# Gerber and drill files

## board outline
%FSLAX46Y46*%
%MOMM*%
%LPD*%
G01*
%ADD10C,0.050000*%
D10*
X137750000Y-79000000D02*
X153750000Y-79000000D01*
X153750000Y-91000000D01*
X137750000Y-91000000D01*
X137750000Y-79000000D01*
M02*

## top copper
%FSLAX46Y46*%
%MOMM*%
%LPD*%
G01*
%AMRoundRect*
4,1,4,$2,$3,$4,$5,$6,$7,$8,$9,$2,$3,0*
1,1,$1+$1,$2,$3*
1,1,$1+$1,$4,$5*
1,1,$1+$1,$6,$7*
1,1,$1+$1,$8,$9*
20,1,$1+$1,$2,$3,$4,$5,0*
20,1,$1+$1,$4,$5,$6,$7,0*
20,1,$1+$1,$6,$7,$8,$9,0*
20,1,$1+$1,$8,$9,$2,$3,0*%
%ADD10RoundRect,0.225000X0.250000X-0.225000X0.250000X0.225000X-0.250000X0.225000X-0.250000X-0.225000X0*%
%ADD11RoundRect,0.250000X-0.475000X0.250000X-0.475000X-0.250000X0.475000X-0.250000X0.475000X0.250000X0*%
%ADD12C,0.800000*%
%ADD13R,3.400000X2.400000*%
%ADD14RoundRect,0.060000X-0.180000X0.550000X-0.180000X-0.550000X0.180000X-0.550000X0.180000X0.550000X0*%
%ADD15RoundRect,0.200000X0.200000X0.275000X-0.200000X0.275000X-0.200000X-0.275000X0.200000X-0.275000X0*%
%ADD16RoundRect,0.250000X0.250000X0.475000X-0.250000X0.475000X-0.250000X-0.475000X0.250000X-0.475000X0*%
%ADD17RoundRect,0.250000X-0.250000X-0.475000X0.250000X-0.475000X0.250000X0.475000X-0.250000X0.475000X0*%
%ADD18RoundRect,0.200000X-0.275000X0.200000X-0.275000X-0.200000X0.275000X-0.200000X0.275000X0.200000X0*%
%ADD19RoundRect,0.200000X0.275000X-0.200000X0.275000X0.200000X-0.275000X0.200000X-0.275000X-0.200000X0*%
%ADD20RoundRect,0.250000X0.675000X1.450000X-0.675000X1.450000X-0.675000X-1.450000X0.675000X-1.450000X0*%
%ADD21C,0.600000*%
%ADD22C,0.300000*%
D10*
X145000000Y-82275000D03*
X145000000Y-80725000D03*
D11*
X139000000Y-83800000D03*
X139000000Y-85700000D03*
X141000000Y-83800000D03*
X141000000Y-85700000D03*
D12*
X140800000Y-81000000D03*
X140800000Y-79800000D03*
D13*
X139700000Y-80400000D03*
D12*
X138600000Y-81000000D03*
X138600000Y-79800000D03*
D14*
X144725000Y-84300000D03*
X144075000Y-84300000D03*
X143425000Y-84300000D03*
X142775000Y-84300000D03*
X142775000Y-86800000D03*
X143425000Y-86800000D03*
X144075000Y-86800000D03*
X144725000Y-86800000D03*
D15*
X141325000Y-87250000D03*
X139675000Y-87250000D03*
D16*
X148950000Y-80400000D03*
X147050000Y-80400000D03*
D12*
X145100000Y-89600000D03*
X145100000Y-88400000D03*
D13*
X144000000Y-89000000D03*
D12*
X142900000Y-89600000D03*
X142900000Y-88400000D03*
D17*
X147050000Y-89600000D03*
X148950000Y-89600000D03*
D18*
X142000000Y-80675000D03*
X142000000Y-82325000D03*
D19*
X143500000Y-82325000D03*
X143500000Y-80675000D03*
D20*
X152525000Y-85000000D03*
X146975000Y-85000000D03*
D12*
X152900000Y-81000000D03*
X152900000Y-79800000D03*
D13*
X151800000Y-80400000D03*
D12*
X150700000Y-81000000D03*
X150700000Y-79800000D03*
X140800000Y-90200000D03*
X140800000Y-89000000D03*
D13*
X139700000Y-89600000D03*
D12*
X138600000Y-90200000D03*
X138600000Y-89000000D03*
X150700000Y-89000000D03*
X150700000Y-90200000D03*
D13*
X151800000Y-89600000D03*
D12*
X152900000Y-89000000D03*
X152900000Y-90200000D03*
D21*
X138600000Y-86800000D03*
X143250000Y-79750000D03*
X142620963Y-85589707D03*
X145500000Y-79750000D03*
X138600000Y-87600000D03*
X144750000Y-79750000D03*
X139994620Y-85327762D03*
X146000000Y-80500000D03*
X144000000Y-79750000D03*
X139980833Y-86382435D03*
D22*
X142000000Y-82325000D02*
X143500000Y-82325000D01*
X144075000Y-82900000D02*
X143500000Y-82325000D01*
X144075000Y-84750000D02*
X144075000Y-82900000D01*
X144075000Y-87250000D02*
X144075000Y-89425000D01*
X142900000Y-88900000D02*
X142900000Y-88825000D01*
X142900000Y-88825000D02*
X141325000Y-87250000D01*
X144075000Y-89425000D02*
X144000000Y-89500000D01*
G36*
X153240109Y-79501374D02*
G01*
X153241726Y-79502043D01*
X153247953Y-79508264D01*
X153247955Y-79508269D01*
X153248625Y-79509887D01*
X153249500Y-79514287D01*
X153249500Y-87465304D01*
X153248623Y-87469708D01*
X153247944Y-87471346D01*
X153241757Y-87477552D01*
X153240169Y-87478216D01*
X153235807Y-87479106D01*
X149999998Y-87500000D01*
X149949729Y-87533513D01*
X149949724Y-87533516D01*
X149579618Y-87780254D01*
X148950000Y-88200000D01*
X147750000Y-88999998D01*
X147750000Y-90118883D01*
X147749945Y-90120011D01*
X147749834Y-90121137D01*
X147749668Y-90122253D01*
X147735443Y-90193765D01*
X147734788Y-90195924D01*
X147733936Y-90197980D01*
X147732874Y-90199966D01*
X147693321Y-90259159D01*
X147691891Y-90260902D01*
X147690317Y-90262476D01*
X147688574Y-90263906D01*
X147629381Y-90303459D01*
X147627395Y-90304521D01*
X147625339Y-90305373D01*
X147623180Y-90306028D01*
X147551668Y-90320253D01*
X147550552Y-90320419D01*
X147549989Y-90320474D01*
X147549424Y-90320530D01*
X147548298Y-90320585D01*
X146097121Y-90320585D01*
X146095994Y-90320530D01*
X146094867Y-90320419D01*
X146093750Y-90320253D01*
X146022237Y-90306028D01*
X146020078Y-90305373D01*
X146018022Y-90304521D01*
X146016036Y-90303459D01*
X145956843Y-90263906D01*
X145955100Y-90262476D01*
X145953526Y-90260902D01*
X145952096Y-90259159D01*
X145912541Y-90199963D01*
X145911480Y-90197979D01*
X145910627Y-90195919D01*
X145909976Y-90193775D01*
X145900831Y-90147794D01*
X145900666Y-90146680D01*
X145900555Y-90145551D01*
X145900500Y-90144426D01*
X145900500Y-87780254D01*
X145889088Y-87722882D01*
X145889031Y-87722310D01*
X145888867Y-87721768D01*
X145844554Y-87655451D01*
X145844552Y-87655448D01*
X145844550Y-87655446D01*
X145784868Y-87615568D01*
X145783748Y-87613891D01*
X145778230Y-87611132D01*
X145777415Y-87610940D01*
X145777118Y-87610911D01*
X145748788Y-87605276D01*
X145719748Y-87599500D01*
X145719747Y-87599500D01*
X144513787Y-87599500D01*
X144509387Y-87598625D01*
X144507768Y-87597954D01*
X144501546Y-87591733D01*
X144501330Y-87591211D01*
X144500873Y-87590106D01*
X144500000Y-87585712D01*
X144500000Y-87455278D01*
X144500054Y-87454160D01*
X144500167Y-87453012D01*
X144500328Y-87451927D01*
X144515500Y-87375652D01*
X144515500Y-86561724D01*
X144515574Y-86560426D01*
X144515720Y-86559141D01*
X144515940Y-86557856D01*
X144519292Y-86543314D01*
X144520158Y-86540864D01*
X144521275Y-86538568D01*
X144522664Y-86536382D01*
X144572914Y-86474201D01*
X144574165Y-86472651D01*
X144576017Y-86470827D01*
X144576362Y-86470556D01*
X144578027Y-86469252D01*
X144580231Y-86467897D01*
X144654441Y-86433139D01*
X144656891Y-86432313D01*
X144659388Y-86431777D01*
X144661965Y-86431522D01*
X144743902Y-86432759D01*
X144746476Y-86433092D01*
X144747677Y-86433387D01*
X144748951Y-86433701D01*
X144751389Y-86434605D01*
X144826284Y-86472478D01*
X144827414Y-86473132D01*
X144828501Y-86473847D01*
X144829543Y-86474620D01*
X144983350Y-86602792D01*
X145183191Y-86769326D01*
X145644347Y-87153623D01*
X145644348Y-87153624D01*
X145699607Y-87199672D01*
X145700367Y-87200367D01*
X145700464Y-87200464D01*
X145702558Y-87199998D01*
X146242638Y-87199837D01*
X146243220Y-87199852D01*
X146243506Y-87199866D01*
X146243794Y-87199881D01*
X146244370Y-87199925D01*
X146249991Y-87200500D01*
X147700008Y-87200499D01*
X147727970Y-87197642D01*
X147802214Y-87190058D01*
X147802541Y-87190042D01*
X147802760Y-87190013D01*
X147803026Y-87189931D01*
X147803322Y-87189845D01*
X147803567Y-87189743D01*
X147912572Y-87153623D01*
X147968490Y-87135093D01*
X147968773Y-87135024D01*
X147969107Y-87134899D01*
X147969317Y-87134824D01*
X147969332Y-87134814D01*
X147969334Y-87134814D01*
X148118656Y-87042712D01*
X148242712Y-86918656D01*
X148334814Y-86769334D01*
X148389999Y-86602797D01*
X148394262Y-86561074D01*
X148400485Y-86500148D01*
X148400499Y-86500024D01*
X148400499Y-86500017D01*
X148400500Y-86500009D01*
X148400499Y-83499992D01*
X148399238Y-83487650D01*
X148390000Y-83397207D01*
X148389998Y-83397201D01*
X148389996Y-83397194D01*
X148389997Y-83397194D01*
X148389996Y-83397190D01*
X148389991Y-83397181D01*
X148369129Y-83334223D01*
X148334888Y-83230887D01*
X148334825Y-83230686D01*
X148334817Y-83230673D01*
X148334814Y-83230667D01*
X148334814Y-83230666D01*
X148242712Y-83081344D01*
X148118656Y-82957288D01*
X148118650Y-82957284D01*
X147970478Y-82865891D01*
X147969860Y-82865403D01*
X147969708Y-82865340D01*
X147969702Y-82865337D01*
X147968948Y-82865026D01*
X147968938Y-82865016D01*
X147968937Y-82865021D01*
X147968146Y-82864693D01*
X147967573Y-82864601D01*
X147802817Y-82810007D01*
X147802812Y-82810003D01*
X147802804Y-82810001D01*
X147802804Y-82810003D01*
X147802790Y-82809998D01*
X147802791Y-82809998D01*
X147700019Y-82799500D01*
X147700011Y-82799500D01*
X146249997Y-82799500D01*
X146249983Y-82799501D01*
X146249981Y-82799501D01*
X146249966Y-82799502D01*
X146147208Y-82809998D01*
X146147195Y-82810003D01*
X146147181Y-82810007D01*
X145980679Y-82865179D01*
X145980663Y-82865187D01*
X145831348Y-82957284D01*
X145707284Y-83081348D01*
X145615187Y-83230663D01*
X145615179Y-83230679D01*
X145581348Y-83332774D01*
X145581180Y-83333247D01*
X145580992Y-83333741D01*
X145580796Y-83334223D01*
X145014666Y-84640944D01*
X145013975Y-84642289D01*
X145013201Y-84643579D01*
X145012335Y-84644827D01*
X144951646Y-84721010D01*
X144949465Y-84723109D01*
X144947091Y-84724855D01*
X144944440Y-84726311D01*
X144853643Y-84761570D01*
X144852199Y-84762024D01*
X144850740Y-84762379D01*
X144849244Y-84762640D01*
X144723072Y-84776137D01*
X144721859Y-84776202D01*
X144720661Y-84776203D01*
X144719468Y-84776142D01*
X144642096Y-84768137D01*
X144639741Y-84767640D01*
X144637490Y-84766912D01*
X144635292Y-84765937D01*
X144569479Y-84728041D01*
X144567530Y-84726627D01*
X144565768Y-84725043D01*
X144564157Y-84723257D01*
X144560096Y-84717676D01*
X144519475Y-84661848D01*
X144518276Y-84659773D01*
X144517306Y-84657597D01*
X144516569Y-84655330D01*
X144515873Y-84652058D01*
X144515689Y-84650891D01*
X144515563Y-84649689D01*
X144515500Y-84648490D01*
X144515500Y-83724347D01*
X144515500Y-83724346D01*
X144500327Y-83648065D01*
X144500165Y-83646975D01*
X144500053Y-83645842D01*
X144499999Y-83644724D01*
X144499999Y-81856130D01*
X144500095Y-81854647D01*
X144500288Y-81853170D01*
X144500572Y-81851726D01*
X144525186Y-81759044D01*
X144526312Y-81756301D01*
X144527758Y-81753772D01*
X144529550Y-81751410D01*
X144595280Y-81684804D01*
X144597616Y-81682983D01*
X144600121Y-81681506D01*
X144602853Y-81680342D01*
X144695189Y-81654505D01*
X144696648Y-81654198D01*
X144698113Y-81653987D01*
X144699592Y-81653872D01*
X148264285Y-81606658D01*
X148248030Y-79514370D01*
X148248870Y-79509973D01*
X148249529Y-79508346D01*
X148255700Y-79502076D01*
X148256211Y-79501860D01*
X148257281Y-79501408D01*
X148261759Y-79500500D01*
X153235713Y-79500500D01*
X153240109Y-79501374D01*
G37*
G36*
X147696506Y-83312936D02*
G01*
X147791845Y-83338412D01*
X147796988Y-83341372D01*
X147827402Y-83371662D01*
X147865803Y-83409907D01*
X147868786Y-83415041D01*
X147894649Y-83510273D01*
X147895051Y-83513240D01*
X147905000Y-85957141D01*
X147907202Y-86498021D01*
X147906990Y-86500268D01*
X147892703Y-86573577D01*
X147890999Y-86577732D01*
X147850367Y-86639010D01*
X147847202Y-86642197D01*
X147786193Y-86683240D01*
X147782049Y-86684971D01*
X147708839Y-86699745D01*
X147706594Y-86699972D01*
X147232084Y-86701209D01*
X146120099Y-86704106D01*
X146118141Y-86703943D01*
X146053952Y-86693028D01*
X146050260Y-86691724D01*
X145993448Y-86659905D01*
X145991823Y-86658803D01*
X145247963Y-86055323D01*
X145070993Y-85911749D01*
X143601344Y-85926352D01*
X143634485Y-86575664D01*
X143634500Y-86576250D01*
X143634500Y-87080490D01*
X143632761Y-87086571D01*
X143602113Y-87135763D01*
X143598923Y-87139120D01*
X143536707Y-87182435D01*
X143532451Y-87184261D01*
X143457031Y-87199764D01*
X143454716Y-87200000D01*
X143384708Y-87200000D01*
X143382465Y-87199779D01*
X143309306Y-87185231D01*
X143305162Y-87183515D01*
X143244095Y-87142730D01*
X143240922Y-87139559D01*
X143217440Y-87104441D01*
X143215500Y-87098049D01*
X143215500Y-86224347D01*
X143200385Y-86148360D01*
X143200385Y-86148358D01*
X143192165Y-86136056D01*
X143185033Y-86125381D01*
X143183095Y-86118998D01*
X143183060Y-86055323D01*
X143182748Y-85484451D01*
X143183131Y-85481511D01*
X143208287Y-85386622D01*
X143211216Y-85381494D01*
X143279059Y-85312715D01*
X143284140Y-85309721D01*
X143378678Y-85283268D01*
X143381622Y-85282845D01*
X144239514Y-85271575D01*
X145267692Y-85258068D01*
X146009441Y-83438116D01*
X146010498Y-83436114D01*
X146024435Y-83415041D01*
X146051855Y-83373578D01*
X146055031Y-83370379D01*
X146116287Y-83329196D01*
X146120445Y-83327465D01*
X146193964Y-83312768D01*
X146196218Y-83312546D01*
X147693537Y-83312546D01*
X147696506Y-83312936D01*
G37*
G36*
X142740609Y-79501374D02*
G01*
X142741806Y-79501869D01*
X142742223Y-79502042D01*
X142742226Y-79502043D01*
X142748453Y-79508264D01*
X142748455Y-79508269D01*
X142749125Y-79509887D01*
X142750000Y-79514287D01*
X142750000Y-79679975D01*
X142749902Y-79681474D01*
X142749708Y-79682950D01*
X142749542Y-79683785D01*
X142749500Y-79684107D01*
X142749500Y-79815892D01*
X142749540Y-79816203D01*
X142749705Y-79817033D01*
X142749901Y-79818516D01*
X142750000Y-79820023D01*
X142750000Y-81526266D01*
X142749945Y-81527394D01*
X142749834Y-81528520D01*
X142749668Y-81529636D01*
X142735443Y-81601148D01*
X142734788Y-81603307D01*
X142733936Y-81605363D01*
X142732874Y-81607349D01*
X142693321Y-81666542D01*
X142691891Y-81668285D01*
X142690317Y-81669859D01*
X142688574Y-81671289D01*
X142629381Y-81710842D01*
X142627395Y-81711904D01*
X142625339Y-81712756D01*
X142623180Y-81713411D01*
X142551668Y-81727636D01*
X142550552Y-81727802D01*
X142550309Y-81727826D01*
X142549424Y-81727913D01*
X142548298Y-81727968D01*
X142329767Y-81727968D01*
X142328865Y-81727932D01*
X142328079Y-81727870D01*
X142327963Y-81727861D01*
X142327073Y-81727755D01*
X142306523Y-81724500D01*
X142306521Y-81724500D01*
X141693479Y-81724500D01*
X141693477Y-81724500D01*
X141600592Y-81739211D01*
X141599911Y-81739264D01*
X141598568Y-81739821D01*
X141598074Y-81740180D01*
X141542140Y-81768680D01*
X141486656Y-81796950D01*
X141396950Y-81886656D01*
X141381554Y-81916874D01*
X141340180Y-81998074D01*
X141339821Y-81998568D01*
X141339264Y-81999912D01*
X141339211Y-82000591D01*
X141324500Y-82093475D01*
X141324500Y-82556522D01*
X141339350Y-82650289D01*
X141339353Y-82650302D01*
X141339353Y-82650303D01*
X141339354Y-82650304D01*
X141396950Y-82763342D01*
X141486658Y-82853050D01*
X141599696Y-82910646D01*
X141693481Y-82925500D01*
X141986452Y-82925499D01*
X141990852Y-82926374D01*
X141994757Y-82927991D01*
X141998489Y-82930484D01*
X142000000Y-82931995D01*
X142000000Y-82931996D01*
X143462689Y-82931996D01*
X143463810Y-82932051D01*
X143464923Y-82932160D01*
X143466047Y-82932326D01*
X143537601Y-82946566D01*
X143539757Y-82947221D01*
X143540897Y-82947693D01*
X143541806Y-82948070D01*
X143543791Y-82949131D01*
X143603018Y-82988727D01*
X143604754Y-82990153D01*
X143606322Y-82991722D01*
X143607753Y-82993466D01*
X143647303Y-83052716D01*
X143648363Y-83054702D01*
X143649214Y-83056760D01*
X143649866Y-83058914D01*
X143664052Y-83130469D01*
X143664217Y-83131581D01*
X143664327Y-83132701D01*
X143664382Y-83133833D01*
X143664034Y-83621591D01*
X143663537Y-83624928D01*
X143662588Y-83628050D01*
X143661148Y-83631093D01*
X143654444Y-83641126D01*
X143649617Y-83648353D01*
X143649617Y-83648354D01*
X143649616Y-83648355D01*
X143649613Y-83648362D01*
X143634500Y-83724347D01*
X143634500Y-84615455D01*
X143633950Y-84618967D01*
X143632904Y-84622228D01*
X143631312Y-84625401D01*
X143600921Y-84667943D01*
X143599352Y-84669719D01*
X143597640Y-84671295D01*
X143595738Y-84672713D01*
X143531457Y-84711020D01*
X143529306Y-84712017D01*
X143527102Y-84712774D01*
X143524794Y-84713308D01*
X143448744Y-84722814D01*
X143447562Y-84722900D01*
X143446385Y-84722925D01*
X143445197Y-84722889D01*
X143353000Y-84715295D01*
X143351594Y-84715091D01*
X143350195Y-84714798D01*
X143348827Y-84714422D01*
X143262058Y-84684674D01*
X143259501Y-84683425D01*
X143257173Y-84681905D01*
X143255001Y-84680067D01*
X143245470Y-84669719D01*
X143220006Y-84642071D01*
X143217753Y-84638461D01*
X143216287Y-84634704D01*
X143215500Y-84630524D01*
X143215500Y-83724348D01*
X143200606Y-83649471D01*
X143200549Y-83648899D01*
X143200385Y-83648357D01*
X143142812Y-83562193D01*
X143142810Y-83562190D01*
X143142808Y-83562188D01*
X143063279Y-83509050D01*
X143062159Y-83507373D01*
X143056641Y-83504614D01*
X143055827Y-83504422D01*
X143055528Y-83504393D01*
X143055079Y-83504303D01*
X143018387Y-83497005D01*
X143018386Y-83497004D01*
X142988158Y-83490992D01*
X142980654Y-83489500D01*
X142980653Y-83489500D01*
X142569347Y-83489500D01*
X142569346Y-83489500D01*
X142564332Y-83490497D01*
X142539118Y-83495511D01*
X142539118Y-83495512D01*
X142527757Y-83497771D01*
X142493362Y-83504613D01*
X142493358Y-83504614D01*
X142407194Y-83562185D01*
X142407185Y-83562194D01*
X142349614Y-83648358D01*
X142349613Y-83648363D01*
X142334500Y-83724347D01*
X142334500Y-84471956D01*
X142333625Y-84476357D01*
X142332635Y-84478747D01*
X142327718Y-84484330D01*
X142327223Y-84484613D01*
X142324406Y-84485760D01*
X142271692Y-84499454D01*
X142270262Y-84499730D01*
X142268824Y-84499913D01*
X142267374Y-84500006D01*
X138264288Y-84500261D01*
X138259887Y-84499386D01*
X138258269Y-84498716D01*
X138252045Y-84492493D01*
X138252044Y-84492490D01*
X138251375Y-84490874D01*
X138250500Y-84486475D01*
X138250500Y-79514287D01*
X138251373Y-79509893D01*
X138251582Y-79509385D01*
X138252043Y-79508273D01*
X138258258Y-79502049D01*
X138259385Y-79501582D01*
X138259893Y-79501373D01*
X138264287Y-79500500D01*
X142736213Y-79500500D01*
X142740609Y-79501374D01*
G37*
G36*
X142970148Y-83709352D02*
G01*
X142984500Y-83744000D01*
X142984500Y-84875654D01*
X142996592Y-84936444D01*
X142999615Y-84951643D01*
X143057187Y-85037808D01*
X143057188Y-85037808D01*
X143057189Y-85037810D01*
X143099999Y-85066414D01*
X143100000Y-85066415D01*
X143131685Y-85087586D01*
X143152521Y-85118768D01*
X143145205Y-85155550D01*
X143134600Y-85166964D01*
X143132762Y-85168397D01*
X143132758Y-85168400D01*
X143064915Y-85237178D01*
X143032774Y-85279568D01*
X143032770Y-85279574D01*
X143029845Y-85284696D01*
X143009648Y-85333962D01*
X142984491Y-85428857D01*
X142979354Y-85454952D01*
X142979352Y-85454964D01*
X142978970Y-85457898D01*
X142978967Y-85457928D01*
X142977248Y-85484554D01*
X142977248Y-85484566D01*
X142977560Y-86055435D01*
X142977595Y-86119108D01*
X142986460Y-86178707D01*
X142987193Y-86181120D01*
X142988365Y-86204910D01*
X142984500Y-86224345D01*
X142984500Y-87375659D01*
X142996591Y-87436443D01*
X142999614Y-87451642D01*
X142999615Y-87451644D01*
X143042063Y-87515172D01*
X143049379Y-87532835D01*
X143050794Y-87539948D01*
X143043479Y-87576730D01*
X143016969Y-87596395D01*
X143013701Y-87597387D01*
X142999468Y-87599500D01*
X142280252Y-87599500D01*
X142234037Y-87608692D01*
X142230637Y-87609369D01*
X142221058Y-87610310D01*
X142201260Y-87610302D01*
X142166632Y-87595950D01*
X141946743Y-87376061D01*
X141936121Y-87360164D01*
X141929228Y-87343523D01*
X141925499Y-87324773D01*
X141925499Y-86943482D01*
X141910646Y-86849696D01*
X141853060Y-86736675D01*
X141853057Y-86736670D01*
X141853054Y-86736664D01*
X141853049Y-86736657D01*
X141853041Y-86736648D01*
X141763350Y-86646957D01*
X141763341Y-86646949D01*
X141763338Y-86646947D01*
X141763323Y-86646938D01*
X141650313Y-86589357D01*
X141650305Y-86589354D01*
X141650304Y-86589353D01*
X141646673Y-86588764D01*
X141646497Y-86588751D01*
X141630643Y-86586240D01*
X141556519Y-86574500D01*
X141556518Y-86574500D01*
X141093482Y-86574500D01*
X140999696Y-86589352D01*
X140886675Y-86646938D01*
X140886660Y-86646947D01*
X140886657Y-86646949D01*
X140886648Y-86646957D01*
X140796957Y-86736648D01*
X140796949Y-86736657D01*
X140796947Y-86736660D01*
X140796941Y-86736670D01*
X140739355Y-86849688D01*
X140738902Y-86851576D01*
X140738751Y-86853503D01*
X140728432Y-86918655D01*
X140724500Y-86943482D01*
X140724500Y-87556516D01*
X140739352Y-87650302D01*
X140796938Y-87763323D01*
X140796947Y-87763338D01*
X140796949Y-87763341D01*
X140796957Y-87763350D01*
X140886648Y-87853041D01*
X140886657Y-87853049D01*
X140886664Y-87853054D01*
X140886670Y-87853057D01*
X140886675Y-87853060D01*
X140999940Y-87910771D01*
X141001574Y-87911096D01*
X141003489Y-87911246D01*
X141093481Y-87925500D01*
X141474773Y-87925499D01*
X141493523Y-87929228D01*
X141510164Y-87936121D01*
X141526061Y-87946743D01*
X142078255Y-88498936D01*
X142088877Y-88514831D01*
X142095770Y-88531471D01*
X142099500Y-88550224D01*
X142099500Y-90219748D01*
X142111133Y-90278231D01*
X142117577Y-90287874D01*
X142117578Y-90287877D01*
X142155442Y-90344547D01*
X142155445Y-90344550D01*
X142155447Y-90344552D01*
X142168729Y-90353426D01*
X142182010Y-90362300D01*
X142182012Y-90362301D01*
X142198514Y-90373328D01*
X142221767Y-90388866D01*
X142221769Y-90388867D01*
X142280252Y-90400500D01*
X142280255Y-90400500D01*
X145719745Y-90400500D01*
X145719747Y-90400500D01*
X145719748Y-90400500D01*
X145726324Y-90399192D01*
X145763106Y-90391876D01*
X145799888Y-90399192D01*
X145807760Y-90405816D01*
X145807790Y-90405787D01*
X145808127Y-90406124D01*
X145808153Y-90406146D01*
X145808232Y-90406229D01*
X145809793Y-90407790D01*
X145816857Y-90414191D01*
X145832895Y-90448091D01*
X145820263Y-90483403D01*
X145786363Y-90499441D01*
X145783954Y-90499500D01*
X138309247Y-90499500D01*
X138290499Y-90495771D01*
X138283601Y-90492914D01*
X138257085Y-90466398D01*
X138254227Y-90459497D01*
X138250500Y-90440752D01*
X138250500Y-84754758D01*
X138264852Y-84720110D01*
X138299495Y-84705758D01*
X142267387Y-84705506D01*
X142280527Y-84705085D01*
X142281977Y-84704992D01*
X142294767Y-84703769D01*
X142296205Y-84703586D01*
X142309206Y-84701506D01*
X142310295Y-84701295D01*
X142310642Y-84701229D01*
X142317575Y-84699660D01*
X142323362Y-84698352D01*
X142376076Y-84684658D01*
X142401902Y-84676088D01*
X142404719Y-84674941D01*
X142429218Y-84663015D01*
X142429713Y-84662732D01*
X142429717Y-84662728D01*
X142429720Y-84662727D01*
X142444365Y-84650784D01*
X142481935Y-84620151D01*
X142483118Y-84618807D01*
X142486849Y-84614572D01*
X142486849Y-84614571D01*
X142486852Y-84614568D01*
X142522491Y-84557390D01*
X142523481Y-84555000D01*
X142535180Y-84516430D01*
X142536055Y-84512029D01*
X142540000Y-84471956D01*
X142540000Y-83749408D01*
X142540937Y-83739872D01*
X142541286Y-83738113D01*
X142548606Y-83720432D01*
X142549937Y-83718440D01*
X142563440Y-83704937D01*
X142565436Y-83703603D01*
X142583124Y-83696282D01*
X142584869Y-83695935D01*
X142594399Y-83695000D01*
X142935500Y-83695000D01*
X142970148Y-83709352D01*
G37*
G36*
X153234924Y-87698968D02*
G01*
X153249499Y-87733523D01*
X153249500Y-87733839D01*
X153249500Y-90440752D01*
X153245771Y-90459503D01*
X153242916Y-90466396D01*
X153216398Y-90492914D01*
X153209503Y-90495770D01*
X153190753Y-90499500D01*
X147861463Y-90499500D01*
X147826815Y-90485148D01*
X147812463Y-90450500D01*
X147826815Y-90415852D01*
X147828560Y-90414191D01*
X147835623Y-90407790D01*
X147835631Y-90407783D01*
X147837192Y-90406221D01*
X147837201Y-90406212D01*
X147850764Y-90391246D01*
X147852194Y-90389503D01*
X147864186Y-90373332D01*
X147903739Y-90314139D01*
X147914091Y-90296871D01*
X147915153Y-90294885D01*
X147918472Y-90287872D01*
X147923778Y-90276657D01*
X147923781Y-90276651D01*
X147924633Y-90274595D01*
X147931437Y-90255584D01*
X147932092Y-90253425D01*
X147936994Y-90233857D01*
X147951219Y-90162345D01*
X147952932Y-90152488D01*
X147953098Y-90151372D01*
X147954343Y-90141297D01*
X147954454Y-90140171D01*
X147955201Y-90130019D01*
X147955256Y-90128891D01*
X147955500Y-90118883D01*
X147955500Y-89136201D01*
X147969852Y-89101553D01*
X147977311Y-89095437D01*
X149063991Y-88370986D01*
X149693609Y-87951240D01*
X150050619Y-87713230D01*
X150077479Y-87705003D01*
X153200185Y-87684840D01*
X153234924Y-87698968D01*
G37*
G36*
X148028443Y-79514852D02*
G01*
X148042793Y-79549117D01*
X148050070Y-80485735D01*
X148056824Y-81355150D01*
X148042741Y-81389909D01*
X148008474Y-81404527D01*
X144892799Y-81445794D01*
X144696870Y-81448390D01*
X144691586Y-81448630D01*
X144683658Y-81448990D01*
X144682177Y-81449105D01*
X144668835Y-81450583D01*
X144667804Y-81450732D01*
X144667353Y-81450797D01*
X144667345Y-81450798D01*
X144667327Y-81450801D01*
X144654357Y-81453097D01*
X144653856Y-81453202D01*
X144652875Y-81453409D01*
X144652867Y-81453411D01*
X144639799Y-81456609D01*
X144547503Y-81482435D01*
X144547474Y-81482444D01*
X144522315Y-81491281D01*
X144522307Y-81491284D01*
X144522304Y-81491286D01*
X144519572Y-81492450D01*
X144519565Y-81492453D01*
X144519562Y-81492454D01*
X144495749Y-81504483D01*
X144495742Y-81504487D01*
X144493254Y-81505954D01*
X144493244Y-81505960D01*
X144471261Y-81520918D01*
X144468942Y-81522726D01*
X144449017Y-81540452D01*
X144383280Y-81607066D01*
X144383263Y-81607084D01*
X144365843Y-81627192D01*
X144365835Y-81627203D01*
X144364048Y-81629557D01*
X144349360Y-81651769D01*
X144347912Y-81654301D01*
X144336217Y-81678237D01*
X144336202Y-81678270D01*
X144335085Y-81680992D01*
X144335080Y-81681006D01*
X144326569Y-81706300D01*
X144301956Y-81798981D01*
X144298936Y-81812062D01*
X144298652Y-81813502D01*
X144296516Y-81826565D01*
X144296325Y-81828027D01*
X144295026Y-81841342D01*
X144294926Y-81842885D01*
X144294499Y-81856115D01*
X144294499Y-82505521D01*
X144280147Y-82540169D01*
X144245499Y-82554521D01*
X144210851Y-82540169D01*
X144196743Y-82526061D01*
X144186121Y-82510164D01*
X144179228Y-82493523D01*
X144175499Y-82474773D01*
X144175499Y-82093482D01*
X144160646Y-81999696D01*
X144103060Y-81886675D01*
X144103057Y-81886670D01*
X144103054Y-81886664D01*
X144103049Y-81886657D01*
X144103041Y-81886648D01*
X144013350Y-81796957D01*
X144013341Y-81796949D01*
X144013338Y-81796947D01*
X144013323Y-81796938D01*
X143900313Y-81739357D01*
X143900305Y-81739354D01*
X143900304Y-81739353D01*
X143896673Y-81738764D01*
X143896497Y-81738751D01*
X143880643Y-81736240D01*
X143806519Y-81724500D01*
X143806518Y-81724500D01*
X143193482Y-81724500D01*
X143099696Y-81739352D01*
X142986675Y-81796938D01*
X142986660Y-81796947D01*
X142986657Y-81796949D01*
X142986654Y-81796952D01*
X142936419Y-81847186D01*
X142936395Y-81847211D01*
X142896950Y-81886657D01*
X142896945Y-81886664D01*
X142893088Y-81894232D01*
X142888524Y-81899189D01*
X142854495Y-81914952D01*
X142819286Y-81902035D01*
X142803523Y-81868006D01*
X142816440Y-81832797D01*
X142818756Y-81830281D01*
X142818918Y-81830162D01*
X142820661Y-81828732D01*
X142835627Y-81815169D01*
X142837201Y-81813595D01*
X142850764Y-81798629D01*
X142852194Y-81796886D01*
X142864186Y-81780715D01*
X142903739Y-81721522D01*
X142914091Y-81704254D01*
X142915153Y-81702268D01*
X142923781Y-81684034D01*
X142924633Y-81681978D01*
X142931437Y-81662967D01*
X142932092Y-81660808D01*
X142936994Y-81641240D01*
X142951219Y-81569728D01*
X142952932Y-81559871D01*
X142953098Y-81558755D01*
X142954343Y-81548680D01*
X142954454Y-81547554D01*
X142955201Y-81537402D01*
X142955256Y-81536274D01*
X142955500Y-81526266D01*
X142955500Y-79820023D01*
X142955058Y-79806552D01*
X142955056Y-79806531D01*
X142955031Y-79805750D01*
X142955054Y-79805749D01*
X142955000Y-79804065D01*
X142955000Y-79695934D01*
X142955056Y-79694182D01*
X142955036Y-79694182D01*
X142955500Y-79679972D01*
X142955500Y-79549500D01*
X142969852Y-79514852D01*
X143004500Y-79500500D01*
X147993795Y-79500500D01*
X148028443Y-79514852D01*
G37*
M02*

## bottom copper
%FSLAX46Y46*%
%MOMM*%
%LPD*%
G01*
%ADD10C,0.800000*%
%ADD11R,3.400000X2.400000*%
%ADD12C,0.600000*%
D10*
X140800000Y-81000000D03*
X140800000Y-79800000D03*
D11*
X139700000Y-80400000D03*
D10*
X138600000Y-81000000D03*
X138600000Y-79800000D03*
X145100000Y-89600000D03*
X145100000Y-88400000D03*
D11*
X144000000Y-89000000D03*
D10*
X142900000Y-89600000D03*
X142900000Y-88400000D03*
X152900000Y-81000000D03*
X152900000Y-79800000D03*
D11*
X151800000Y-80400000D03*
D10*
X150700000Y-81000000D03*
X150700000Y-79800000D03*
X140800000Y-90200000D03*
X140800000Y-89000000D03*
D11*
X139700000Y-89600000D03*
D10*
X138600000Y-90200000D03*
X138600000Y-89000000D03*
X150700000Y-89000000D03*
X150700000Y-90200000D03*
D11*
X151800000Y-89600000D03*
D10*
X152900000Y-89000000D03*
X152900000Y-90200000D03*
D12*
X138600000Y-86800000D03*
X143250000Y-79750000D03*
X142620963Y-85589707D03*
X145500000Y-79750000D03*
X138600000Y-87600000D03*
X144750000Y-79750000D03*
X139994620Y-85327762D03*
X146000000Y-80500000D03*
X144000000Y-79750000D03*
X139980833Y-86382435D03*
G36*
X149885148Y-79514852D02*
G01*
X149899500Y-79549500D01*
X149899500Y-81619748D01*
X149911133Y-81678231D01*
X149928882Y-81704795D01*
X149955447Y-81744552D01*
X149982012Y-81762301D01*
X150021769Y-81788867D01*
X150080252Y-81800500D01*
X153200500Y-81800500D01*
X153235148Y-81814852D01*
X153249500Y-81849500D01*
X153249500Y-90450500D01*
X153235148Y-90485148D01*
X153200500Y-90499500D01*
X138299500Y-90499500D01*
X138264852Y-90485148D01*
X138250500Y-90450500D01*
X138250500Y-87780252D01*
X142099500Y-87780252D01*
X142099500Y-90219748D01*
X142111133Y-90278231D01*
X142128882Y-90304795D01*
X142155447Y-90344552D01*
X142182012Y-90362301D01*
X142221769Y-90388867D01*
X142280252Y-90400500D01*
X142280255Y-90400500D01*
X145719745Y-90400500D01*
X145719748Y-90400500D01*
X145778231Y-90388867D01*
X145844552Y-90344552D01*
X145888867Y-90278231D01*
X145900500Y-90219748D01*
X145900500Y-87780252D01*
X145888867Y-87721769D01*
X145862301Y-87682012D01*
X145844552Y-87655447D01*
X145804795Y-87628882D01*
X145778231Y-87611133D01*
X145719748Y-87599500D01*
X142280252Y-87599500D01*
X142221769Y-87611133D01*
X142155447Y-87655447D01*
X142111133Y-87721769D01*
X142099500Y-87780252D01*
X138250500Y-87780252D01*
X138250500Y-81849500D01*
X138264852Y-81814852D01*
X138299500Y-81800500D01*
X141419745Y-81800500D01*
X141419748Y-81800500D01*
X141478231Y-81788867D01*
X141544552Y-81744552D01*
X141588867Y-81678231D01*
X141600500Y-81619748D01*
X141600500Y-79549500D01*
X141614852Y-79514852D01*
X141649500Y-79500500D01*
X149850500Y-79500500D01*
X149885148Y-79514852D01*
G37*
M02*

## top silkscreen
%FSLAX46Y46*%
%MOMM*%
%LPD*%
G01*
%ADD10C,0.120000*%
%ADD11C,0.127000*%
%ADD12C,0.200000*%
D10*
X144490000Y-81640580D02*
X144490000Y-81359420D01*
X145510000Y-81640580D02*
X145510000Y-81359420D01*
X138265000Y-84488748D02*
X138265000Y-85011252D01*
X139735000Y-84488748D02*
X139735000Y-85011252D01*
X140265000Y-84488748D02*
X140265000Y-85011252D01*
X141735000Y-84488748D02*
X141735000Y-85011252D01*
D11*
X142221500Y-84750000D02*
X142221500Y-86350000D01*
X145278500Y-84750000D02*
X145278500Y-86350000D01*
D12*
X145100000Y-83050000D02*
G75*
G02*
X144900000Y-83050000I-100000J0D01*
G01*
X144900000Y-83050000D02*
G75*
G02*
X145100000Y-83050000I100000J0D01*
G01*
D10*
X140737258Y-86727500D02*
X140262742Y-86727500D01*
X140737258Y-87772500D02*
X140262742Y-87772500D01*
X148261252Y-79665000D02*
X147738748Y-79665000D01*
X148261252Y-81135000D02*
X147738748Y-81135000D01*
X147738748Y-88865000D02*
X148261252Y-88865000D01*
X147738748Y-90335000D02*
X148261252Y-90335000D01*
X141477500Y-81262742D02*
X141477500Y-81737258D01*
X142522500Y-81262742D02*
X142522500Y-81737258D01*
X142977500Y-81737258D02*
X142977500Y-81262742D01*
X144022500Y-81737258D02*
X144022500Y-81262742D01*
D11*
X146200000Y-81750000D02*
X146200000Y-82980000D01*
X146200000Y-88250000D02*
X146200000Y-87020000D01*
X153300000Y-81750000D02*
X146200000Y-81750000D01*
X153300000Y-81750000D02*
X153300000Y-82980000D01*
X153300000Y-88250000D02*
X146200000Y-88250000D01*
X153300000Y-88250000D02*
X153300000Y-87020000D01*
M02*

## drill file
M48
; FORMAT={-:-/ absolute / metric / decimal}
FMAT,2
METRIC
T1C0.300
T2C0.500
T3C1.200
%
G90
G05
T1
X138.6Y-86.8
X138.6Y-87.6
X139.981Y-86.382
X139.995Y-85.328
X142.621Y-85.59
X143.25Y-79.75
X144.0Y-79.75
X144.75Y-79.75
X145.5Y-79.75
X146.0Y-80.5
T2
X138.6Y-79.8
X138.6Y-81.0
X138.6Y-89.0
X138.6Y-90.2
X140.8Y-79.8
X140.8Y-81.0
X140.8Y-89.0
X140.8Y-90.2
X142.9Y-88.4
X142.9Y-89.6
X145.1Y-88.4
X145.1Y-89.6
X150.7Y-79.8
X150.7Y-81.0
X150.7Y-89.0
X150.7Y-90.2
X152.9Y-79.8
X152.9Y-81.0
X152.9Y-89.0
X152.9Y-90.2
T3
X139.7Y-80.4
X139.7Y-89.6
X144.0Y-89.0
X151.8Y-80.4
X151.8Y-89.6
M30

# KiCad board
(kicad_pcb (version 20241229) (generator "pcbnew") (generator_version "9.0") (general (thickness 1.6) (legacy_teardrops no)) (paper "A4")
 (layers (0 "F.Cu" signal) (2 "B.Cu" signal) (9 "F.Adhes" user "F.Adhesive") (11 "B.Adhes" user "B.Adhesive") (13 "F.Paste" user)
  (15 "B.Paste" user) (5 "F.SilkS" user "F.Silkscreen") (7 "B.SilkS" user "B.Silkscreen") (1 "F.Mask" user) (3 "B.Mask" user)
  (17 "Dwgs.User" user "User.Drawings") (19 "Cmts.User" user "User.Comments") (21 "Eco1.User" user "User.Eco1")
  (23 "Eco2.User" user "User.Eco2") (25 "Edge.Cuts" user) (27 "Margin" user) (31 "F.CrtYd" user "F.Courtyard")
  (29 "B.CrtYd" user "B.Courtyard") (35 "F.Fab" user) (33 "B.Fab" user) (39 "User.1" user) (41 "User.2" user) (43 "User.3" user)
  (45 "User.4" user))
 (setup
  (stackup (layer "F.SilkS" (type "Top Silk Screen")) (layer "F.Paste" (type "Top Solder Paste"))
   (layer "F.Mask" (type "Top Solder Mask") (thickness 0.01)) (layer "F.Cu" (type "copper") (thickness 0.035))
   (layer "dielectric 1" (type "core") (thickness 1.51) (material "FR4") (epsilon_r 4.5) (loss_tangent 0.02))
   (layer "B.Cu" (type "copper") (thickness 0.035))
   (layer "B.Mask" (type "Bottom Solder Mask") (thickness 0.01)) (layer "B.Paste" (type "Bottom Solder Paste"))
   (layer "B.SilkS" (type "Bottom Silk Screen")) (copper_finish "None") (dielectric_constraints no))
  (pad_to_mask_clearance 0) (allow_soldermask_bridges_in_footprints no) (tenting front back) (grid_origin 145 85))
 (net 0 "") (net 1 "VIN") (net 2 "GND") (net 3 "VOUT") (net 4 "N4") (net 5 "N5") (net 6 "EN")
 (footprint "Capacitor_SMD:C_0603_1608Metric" (layer "F.Cu") (at 145 81.5 90)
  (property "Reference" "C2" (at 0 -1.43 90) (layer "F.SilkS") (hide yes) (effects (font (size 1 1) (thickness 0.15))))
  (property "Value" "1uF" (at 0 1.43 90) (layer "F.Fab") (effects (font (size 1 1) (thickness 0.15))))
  (fp_line (start -0.14058 -0.51) (end 0.14058 -0.51) (stroke (width 0.12) (type solid)) (layer "F.SilkS"))
  (fp_line (start -0.14058 0.51) (end 0.14058 0.51) (stroke (width 0.12) (type solid)) (layer "F.SilkS"))
  (pad "1" smd roundrect (at -0.775 0 90) (size 0.9 0.95) (layers "F.Cu" "F.Mask" "F.Paste") (roundrect_rratio 0.25) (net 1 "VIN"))
  (pad "2" smd roundrect (at 0.775 0 90) (size 0.9 0.95) (layers "F.Cu" "F.Mask" "F.Paste") (roundrect_rratio 0.25) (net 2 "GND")))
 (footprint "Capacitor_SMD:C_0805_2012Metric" (layer "F.Cu") (at 139 84.75 -90)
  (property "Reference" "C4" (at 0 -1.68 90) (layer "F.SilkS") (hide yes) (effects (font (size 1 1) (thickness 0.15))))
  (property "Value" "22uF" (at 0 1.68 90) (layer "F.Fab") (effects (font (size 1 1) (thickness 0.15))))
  (fp_line (start -0.261252 0.735) (end 0.261252 0.735) (stroke (width 0.12) (type solid)) (layer "F.SilkS"))
  (fp_line (start -0.261252 -0.735) (end 0.261252 -0.735) (stroke (width 0.12) (type solid)) (layer "F.SilkS"))
  (pad "1" smd roundrect (at -0.95 0 270) (size 1 1.45) (layers "F.Cu" "F.Mask" "F.Paste") (roundrect_rratio 0.25) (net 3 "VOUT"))
  (pad "2" smd roundrect (at 0.95 0 270) (size 1 1.45) (layers "F.Cu" "F.Mask" "F.Paste") (roundrect_rratio 0.25) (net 2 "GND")))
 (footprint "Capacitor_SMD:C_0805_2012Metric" (layer "F.Cu") (at 141 84.75 -90)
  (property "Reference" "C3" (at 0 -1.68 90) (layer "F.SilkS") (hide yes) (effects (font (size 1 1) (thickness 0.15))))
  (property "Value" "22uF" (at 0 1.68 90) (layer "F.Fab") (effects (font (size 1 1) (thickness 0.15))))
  (fp_line (start -0.261252 0.735) (end 0.261252 0.735) (stroke (width 0.12) (type solid)) (layer "F.SilkS"))
  (fp_line (start -0.261252 -0.735) (end 0.261252 -0.735) (stroke (width 0.12) (type solid)) (layer "F.SilkS"))
  (pad "1" smd roundrect (at -0.95 0 270) (size 1 1.45) (layers "F.Cu" "F.Mask" "F.Paste") (roundrect_rratio 0.25) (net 3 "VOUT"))
  (pad "2" smd roundrect (at 0.95 0 270) (size 1 1.45) (layers "F.Cu" "F.Mask" "F.Paste") (roundrect_rratio 0.25) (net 2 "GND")))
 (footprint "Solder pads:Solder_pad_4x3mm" (layer "F.Cu") (at 139.7 80.4 180)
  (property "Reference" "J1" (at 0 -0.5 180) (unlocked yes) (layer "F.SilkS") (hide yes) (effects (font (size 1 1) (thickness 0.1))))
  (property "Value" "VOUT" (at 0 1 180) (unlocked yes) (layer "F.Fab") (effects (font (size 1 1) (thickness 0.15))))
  (pad "1" thru_hole circle (at -1.1 -0.6 180) (size 0.8 0.8) (drill 0.5) (layers "*.Cu" "*.Mask") (remove_unused_layers no) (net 3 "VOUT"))
  (pad "1" thru_hole circle (at -1.1 0.6 180) (size 0.8 0.8) (drill 0.5) (layers "*.Cu" "*.Mask") (remove_unused_layers no) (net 3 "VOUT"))
  (pad "1" thru_hole rect (at 0 0 180) (size 3.4 2.4) (drill 1.2) (layers "*.Cu" "*.Mask") (remove_unused_layers no) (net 3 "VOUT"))
  (pad "1" thru_hole circle (at 1.1 -0.6 180) (size 0.8 0.8) (drill 0.5) (layers "*.Cu" "*.Mask") (remove_unused_layers no) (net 3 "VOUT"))
  (pad "1" thru_hole circle (at 1.1 0.6 180) (size 0.8 0.8) (drill 0.5) (layers "*.Cu" "*.Mask") (remove_unused_layers no) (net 3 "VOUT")))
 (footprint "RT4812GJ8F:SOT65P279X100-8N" (layer "F.Cu") (at 143.75 85.55 -90)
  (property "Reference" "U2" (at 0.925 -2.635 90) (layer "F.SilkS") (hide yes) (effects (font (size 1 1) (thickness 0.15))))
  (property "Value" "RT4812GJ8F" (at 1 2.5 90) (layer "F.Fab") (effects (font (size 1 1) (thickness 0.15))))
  (fp_line (start -0.8 1.5285) (end 0.8 1.5285) (stroke (width 0.127) (type solid)) (layer "F.SilkS"))
  (fp_line (start -0.8 -1.5285) (end 0.8 -1.5285) (stroke (width 0.127) (type solid)) (layer "F.SilkS"))
  (fp_circle (center -2.5 -1.25) (end -2.4 -1.25) (stroke (width 0.2) (type solid)) (fill no) (layer "F.SilkS"))
  (pad "1" smd roundrect (at -1.25 -0.975 270) (size 1.22 0.48) (layers "F.Cu" "F.Mask" "F.Paste") (roundrect_rratio 0.125) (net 1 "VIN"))
  (pad "2" smd roundrect (at -1.25 -0.325 270) (size 1.22 0.48) (layers "F.Cu" "F.Mask" "F.Paste") (roundrect_rratio 0.125) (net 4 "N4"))
  (pad "3" smd roundrect (at -1.25 0.325 270) (size 1.22 0.48) (layers "F.Cu" "F.Mask" "F.Paste") (roundrect_rratio 0.125) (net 3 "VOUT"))
  (pad "4" smd roundrect (at -1.25 0.975 270) (size 1.22 0.48) (layers "F.Cu" "F.Mask" "F.Paste") (roundrect_rratio 0.125) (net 2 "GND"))
  (pad "5" smd roundrect (at 1.25 0.975 270) (size 1.22 0.48) (layers "F.Cu" "F.Mask" "F.Paste") (roundrect_rratio 0.125) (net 2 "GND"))
  (pad "6" smd roundrect (at 1.25 0.325 270) (size 1.22 0.48) (layers "F.Cu" "F.Mask" "F.Paste") (roundrect_rratio 0.125) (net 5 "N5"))
  (pad "7" smd roundrect (at 1.25 -0.325 270) (size 1.22 0.48) (layers "F.Cu" "F.Mask" "F.Paste") (roundrect_rratio 0.125) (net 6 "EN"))
  (pad "8" smd roundrect (at 1.25 -0.975 270) (size 1.22 0.48) (layers "F.Cu" "F.Mask" "F.Paste") (roundrect_rratio 0.125) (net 1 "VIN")))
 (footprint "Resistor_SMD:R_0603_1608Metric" (layer "F.Cu") (at 140.5 87.25 180)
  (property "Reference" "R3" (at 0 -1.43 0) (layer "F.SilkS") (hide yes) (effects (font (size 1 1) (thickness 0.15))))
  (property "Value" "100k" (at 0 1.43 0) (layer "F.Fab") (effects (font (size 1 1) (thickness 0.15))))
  (fp_line (start -0.237258 0.5225) (end 0.237258 0.5225) (stroke (width 0.12) (type solid)) (layer "F.SilkS"))
  (fp_line (start -0.237258 -0.5225) (end 0.237258 -0.5225) (stroke (width 0.12) (type solid)) (layer "F.SilkS"))
  (pad "1" smd roundrect (at -0.825 0 180) (size 0.8 0.95) (layers "F.Cu" "F.Mask" "F.Paste") (roundrect_rratio 0.25) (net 6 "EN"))
  (pad "2" smd roundrect (at 0.825 0 180) (size 0.8 0.95) (layers "F.Cu" "F.Mask" "F.Paste") (roundrect_rratio 0.25) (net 2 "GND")))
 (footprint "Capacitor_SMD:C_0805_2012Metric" (layer "F.Cu") (at 148 80.4 180)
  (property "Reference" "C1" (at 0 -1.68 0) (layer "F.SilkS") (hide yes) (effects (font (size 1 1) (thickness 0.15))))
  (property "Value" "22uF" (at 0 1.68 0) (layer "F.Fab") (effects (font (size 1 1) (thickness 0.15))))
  (fp_line (start -0.261252 0.735) (end 0.261252 0.735) (stroke (width 0.12) (type solid)) (layer "F.SilkS"))
  (fp_line (start -0.261252 -0.735) (end 0.261252 -0.735) (stroke (width 0.12) (type solid)) (layer "F.SilkS"))
  (pad "1" smd roundrect (at -0.95 0 180) (size 1 1.45) (layers "F.Cu" "F.Mask" "F.Paste") (roundrect_rratio 0.25) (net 1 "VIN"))
  (pad "2" smd roundrect (at 0.95 0 180) (size 1 1.45) (layers "F.Cu" "F.Mask" "F.Paste") (roundrect_rratio 0.25) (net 2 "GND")))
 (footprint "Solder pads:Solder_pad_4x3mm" (layer "F.Cu") (at 144 89 180)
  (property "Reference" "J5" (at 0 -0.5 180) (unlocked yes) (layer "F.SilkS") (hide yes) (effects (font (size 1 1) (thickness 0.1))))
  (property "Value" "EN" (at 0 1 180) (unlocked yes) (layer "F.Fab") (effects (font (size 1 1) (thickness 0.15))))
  (pad "1" thru_hole circle (at -1.1 -0.6 180) (size 0.8 0.8) (drill 0.5) (layers "*.Cu" "*.Mask") (remove_unused_layers no) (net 6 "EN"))
  (pad "1" thru_hole circle (at -1.1 0.6 180) (size 0.8 0.8) (drill 0.5) (layers "*.Cu" "*.Mask") (remove_unused_layers no) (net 6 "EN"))
  (pad "1" thru_hole rect (at 0 0 180) (size 3.4 2.4) (drill 1.2) (layers "*.Cu" "*.Mask") (remove_unused_layers no) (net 6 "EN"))
  (pad "1" thru_hole circle (at 1.1 -0.6 180) (size 0.8 0.8) (drill 0.5) (layers "*.Cu" "*.Mask") (remove_unused_layers no) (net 6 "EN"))
  (pad "1" thru_hole circle (at 1.1 0.6 180) (size 0.8 0.8) (drill 0.5) (layers "*.Cu" "*.Mask") (remove_unused_layers no) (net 6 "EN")))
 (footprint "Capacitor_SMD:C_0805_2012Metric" (layer "F.Cu") (at 148 89.6)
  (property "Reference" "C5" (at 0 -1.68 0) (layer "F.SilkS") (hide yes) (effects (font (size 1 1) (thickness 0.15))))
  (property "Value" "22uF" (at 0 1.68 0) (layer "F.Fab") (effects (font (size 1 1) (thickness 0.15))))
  (fp_line (start -0.261252 -0.735) (end 0.261252 -0.735) (stroke (width 0.12) (type solid)) (layer "F.SilkS"))
  (fp_line (start -0.261252 0.735) (end 0.261252 0.735) (stroke (width 0.12) (type solid)) (layer "F.SilkS"))
  (pad "1" smd roundrect (at -0.95 0) (size 1 1.45) (layers "F.Cu" "F.Mask" "F.Paste") (roundrect_rratio 0.25) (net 1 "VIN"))
  (pad "2" smd roundrect (at 0.95 0) (size 1 1.45) (layers "F.Cu" "F.Mask" "F.Paste") (roundrect_rratio 0.25) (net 2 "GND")))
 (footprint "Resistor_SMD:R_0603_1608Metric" (layer "F.Cu") (at 142 81.5 -90)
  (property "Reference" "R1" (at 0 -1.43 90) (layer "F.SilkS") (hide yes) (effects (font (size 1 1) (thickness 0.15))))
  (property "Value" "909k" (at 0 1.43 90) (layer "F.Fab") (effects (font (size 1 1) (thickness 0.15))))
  (fp_line (start -0.237258 0.5225) (end 0.237258 0.5225) (stroke (width 0.12) (type solid)) (layer "F.SilkS"))
  (fp_line (start -0.237258 -0.5225) (end 0.237258 -0.5225) (stroke (width 0.12) (type solid)) (layer "F.SilkS"))
  (pad "1" smd roundrect (at -0.825 0 270) (size 0.8 0.95) (layers "F.Cu" "F.Mask" "F.Paste") (roundrect_rratio 0.25) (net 3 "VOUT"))
  (pad "2" smd roundrect (at 0.825 0 270) (size 0.8 0.95) (layers "F.Cu" "F.Mask" "F.Paste") (roundrect_rratio 0.25) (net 4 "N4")))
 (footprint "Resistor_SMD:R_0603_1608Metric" (layer "F.Cu") (at 143.5 81.5 90)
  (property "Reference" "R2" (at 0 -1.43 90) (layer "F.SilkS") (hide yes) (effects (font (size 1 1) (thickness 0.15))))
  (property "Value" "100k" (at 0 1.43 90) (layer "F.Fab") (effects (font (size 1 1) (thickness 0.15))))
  (fp_line (start -0.237258 -0.5225) (end 0.237258 -0.5225) (stroke (width 0.12) (type solid)) (layer "F.SilkS"))
  (fp_line (start -0.237258 0.5225) (end 0.237258 0.5225) (stroke (width 0.12) (type solid)) (layer "F.SilkS"))
  (pad "1" smd roundrect (at -0.825 0 90) (size 0.8 0.95) (layers "F.Cu" "F.Mask" "F.Paste") (roundrect_rratio 0.25) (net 4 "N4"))
  (pad "2" smd roundrect (at 0.825 0 90) (size 0.8 0.95) (layers "F.Cu" "F.Mask" "F.Paste") (roundrect_rratio 0.25) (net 2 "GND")))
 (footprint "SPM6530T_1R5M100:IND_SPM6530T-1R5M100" (layer "F.Cu") (at 149.75 85 180)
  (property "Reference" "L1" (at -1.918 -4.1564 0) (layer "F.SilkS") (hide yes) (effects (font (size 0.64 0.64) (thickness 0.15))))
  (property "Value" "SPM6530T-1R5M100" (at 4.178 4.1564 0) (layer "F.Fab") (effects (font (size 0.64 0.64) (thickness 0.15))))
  (fp_line (start 3.55 3.25) (end 3.55 2.02) (stroke (width 0.127) (type solid)) (layer "F.SilkS"))
  (fp_line (start 3.55 -3.25) (end 3.55 -2.02) (stroke (width 0.127) (type solid)) (layer "F.SilkS"))
  (fp_line (start -3.55 3.25) (end 3.55 3.25) (stroke (width 0.127) (type solid)) (layer "F.SilkS"))
  (fp_line (start -3.55 3.25) (end -3.55 2.02) (stroke (width 0.127) (type solid)) (layer "F.SilkS"))
  (fp_line (start -3.55 -3.25) (end 3.55 -3.25) (stroke (width 0.127) (type solid)) (layer "F.SilkS"))
  (fp_line (start -3.55 -3.25) (end -3.55 -2.02) (stroke (width 0.127) (type solid)) (layer "F.SilkS"))
  (pad "1" smd roundrect (at -2.775 0 180) (size 1.85 3.4) (layers "F.Cu" "F.Mask" "F.Paste") (roundrect_rratio 0.1351351351) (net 1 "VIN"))
  (pad "2" smd roundrect (at 2.775 0 180) (size 1.85 3.4) (layers "F.Cu" "F.Mask" "F.Paste") (roundrect_rratio 0.1351351351) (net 5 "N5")
   (clearance 0.5)))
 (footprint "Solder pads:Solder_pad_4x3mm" (layer "F.Cu") (at 151.8 80.4 180)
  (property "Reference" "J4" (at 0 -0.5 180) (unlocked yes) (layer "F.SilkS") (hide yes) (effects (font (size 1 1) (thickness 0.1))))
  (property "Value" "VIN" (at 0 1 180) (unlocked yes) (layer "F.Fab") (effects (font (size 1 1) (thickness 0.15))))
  (pad "1" thru_hole circle (at -1.1 -0.6 180) (size 0.8 0.8) (drill 0.5) (layers "*.Cu" "*.Mask") (remove_unused_layers no) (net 1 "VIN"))
  (pad "1" thru_hole circle (at -1.1 0.6 180) (size 0.8 0.8) (drill 0.5) (layers "*.Cu" "*.Mask") (remove_unused_layers no) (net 1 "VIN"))
  (pad "1" thru_hole rect (at 0 0 180) (size 3.4 2.4) (drill 1.2) (layers "*.Cu" "*.Mask") (remove_unused_layers no) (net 1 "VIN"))
  (pad "1" thru_hole circle (at 1.1 -0.6 180) (size 0.8 0.8) (drill 0.5) (layers "*.Cu" "*.Mask") (remove_unused_layers no) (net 1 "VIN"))
  (pad "1" thru_hole circle (at 1.1 0.6 180) (size 0.8 0.8) (drill 0.5) (layers "*.Cu" "*.Mask") (remove_unused_layers no) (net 1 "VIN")))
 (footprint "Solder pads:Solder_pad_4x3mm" (layer "F.Cu") (at 139.7 89.6 180)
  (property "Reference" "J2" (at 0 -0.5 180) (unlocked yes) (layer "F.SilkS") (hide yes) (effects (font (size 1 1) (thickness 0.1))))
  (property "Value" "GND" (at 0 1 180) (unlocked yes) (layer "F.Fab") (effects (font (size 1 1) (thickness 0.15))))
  (pad "1" thru_hole circle (at -1.1 -0.6 180) (size 0.8 0.8) (drill 0.5) (layers "*.Cu" "*.Mask") (remove_unused_layers no) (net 2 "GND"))
  (pad "1" thru_hole circle (at -1.1 0.6 180) (size 0.8 0.8) (drill 0.5) (layers "*.Cu" "*.Mask") (remove_unused_layers no) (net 2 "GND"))
  (pad "1" thru_hole rect (at 0 0 180) (size 3.4 2.4) (drill 1.2) (layers "*.Cu" "*.Mask") (remove_unused_layers no) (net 2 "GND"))
  (pad "1" thru_hole circle (at 1.1 -0.6 180) (size 0.8 0.8) (drill 0.5) (layers "*.Cu" "*.Mask") (remove_unused_layers no) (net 2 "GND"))
  (pad "1" thru_hole circle (at 1.1 0.6 180) (size 0.8 0.8) (drill 0.5) (layers "*.Cu" "*.Mask") (remove_unused_layers no) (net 2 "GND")))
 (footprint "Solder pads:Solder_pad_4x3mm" (layer "F.Cu") (at 151.8 89.6)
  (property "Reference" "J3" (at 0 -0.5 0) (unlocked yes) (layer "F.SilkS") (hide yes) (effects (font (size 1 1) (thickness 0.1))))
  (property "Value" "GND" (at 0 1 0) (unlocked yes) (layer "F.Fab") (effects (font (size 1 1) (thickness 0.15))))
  (pad "1" thru_hole circle (at -1.1 -0.6) (size 0.8 0.8) (drill 0.5) (layers "*.Cu" "*.Mask") (remove_unused_layers no) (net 2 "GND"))
  (pad "1" thru_hole circle (at -1.1 0.6) (size 0.8 0.8) (drill 0.5) (layers "*.Cu" "*.Mask") (remove_unused_layers no) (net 2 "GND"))
  (pad "1" thru_hole rect (at 0 0) (size 3.4 2.4) (drill 1.2) (layers "*.Cu" "*.Mask") (remove_unused_layers no) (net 2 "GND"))
  (pad "1" thru_hole circle (at 1.1 -0.6) (size 0.8 0.8) (drill 0.5) (layers "*.Cu" "*.Mask") (remove_unused_layers no) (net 2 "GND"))
  (pad "1" thru_hole circle (at 1.1 0.6) (size 0.8 0.8) (drill 0.5) (layers "*.Cu" "*.Mask") (remove_unused_layers no) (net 2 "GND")))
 (gr_rect (start 137.75 79) (end 153.75 91) (stroke (width 0.05) (type solid)) (fill no) (layer "Edge.Cuts"))
 (via (at 138.6 86.8) (size 0.6) (drill 0.3) (layers "F.Cu" "B.Cu") (free yes) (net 2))
 (via (at 143.25 79.75) (size 0.6) (drill 0.3) (layers "F.Cu" "B.Cu") (free yes) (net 2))
 (via (at 142.620963 85.589707) (size 0.6) (drill 0.3) (layers "F.Cu" "B.Cu") (free yes) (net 2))
 (via (at 145.5 79.75) (size 0.6) (drill 0.3) (layers "F.Cu" "B.Cu") (free yes) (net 2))
 (via (at 138.6 87.6) (size 0.6) (drill 0.3) (layers "F.Cu" "B.Cu") (free yes) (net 2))
 (via (at 144.75 79.75) (size 0.6) (drill 0.3) (layers "F.Cu" "B.Cu") (free yes) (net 2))
 (via (at 139.99462 85.327762) (size 0.6) (drill 0.3) (layers "F.Cu" "B.Cu") (free yes) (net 2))
 (via (at 146 80.5) (size 0.6) (drill 0.3) (layers "F.Cu" "B.Cu") (free yes) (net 2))
 (via (at 144 79.75) (size 0.6) (drill 0.3) (layers "F.Cu" "B.Cu") (free yes) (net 2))
 (via (at 139.980833 86.382435) (size 0.6) (drill 0.3) (layers "F.Cu" "B.Cu") (free yes) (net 2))
 (segment (start 142 82.325) (end 143.5 82.325) (width 0.3) (layer "F.Cu") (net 4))
 (segment (start 144.075 82.9) (end 143.5 82.325) (width 0.3) (layer "F.Cu") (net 4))
 (segment (start 144.075 84.75) (end 144.075 82.9) (width 0.3) (layer "F.Cu") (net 4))
 (segment (start 144.075 87.25) (end 144.075 89.425) (width 0.3) (layer "F.Cu") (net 6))
 (segment (start 142.9 88.9) (end 142.9 88.825) (width 0.3) (layer "F.Cu") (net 6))
 (segment (start 142.9 88.825) (end 141.325 87.25) (width 0.3) (layer "F.Cu") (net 6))
 (segment (start 144.075 89.425) (end 144 89.5) (width 0.3) (layer "F.Cu") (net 6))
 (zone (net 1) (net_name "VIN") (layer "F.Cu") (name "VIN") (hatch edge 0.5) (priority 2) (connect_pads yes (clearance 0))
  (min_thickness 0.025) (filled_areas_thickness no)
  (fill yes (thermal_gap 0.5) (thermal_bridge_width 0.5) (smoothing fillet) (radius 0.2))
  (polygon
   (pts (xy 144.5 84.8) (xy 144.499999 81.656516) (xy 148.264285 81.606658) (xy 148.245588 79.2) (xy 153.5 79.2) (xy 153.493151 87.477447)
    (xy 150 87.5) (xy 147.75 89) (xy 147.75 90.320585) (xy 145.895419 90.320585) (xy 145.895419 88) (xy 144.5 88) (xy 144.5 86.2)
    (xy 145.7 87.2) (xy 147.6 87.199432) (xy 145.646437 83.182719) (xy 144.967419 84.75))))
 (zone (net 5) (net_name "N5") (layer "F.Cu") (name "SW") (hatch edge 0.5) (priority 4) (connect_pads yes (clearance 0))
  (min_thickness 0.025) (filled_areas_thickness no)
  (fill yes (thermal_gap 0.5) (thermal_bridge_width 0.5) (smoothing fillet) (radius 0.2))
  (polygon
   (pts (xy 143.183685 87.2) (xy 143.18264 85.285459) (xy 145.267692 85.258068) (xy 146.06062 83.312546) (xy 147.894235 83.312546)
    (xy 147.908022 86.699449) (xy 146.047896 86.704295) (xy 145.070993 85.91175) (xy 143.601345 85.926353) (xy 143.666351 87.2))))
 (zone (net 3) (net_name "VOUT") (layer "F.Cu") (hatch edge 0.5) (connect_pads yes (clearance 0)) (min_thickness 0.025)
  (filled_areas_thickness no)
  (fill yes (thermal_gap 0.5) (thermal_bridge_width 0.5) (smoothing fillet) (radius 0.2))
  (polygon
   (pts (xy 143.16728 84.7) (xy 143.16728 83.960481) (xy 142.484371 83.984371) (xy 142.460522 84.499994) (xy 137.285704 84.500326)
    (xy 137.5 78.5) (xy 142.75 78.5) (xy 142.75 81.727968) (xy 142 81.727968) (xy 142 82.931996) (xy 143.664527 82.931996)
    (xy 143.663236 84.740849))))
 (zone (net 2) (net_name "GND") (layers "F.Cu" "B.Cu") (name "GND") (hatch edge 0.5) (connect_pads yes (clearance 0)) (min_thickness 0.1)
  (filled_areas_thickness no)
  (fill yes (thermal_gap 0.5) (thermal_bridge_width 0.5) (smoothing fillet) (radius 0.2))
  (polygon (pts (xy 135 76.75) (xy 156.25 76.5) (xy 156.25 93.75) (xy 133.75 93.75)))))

